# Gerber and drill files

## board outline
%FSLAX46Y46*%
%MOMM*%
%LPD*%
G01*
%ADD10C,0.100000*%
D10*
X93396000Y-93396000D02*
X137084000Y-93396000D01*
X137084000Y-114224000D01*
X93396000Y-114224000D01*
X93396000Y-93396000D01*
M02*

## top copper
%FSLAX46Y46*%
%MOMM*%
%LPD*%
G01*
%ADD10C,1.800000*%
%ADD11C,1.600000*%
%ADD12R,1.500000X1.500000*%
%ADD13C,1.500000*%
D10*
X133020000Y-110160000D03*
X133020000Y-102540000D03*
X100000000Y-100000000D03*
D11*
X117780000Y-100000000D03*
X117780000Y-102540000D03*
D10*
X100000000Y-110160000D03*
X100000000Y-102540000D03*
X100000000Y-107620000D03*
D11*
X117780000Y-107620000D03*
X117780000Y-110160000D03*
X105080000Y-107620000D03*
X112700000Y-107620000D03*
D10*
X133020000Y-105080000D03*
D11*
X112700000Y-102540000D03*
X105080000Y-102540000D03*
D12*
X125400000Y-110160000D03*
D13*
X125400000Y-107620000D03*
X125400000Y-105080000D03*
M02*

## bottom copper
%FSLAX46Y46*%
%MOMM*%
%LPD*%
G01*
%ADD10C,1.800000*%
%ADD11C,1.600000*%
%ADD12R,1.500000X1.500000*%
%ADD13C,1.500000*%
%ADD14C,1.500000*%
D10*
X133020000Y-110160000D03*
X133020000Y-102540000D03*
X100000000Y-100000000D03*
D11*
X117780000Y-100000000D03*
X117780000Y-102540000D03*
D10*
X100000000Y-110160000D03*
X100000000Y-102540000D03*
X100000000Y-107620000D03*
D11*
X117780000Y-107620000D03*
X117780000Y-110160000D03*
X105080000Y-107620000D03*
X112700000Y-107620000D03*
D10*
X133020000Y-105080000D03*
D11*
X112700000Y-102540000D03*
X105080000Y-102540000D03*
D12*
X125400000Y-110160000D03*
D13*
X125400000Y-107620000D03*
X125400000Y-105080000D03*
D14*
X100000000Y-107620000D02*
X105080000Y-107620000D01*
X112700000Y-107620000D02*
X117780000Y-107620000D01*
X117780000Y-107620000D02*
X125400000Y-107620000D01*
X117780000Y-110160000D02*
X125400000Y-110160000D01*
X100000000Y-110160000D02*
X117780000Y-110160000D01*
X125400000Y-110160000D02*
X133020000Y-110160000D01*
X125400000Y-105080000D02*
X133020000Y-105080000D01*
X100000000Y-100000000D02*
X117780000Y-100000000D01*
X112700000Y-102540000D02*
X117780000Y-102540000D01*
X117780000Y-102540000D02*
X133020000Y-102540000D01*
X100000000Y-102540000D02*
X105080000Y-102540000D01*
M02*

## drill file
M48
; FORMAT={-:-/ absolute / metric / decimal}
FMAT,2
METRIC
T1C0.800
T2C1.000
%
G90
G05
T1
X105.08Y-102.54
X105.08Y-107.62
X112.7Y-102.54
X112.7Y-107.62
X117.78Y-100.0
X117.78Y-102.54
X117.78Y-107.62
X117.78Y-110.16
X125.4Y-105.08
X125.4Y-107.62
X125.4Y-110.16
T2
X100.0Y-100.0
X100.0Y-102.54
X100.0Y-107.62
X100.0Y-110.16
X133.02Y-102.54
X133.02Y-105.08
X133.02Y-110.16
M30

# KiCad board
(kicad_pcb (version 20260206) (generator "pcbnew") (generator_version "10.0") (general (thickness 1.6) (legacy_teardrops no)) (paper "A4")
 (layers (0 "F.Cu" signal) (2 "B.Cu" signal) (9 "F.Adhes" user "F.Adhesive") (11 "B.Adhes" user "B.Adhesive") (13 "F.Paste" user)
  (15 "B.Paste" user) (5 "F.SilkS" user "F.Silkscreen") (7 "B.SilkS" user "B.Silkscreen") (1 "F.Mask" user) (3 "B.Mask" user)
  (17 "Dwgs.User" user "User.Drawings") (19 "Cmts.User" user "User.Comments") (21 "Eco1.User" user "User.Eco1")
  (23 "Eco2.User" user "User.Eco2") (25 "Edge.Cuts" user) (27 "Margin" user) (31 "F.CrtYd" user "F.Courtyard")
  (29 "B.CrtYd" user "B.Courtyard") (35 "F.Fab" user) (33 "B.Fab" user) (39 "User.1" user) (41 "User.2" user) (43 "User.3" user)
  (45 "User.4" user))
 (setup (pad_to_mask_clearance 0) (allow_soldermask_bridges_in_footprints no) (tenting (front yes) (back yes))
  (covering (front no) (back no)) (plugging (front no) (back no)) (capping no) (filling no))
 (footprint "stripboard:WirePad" (layer "F.Cu") (at 133.02 110.16)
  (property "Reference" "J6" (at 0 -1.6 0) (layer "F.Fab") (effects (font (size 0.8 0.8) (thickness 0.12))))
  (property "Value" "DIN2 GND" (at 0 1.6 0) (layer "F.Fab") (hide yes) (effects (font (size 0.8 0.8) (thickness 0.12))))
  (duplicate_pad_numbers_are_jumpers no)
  (pad "1" thru_hole circle (at 0 0) (size 1.8 1.8) (drill 1) (layers "*.Cu" "*.Mask") (remove_unused_layers no) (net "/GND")))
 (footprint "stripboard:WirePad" (layer "F.Cu") (at 133.02 102.54)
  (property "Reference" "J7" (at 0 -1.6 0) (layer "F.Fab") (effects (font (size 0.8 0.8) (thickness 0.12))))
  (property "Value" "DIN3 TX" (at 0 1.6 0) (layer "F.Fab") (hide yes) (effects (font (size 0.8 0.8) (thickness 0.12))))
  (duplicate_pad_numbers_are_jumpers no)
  (pad "1" thru_hole circle (at 0 0) (size 1.8 1.8) (drill 1) (layers "*.Cu" "*.Mask") (remove_unused_layers no) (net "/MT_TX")))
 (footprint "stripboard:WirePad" (layer "F.Cu") (at 100 100)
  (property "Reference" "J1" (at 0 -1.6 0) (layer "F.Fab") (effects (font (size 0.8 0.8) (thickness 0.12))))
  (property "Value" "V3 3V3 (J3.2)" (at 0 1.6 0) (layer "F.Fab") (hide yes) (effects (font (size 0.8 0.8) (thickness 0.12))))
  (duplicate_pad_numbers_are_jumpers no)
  (pad "1" thru_hole circle (at 0 0) (size 1.8 1.8) (drill 1) (layers "*.Cu" "*.Mask") (remove_unused_layers no) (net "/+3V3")))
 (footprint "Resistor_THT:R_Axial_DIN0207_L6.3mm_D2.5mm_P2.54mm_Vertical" (layer "F.Cu") (at 117.78 100 -90)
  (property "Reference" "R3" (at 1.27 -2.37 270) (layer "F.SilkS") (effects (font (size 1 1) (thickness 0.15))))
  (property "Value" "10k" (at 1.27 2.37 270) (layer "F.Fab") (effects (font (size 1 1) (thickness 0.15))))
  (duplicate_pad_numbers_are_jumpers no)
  (pad "1" thru_hole circle (at 0 0 270) (size 1.6 1.6) (drill 0.8) (layers "*.Cu" "*.Mask") (remove_unused_layers no) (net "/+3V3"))
  (pad "2" thru_hole circle (at 2.54 0 270) (size 1.6 1.6) (drill 0.8) (layers "*.Cu" "*.Mask") (remove_unused_layers no) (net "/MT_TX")))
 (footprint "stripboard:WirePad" (layer "F.Cu") (at 100 110.16)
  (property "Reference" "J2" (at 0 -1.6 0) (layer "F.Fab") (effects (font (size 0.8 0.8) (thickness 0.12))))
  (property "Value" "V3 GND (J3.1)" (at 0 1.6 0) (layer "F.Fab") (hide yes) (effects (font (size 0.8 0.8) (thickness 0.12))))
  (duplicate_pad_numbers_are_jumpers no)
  (pad "1" thru_hole circle (at 0 0) (size 1.8 1.8) (drill 1) (layers "*.Cu" "*.Mask") (remove_unused_layers no) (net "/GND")))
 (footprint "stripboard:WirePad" (layer "F.Cu") (at 100 102.54)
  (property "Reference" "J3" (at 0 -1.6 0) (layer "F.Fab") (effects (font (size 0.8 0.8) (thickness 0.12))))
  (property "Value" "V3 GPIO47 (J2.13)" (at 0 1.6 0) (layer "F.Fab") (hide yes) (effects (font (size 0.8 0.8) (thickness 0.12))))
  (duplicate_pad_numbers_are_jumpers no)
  (pad "1" thru_hole circle (at 0 0) (size 1.8 1.8) (drill 1) (layers "*.Cu" "*.Mask") (remove_unused_layers no) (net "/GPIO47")))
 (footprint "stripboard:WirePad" (layer "F.Cu") (at 100 107.62)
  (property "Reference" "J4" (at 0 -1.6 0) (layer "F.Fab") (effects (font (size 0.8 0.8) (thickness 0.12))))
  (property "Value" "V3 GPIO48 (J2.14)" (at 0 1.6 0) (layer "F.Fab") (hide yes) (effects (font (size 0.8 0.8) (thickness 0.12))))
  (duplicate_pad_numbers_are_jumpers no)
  (pad "1" thru_hole circle (at 0 0) (size 1.8 1.8) (drill 1) (layers "*.Cu" "*.Mask") (remove_unused_layers no) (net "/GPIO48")))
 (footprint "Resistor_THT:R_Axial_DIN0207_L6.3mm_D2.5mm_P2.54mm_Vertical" (layer "F.Cu") (at 117.78 107.62 -90)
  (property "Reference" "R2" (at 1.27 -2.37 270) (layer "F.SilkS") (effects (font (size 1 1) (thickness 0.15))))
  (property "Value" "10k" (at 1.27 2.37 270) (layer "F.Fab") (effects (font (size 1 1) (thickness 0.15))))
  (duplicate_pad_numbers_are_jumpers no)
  (pad "1" thru_hole circle (at 0 0 270) (size 1.6 1.6) (drill 0.8) (layers "*.Cu" "*.Mask") (remove_unused_layers no) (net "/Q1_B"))
  (pad "2" thru_hole circle (at 2.54 0 270) (size 1.6 1.6) (drill 0.8) (layers "*.Cu" "*.Mask") (remove_unused_layers no) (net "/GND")))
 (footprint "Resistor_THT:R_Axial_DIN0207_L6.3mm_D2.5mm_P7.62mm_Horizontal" (layer "F.Cu") (at 105.08 107.62)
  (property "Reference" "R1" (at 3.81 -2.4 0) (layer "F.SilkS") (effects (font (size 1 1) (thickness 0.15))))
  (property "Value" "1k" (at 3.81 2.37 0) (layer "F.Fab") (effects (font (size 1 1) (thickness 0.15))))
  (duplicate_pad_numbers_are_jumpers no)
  (pad "1" thru_hole circle (at 0 0) (size 1.6 1.6) (drill 0.8) (layers "*.Cu" "*.Mask") (remove_unused_layers no) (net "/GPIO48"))
  (pad "2" thru_hole circle (at 7.62 0) (size 1.6 1.6) (drill 0.8) (layers "*.Cu" "*.Mask") (remove_unused_layers no) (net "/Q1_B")))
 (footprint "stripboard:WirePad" (layer "F.Cu") (at 133.02 105.08)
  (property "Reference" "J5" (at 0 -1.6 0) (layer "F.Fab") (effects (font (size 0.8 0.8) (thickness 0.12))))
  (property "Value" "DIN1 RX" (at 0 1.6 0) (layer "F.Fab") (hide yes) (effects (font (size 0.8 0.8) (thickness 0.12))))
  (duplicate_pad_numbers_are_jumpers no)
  (pad "1" thru_hole circle (at 0 0) (size 1.8 1.8) (drill 1) (layers "*.Cu" "*.Mask") (remove_unused_layers no) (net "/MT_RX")))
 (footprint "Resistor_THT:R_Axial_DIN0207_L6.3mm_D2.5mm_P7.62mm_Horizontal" (layer "F.Cu") (at 112.7 102.54 180)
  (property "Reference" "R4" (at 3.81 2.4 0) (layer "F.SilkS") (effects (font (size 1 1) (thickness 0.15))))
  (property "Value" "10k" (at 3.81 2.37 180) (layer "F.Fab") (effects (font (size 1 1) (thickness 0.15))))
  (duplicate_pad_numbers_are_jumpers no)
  (pad "1" thru_hole circle (at 0 0 180) (size 1.6 1.6) (drill 0.8) (layers "*.Cu" "*.Mask") (remove_unused_layers no) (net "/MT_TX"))
  (pad "2" thru_hole circle (at 7.62 0 180) (size 1.6 1.6) (drill 0.8) (layers "*.Cu" "*.Mask") (remove_unused_layers no) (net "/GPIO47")))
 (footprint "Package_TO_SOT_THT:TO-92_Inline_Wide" (layer "F.Cu") (at 125.4 110.16 90)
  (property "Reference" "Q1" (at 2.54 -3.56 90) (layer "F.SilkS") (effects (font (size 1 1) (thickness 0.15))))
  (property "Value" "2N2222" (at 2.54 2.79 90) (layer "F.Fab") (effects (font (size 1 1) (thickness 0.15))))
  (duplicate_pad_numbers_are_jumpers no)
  (pad "1" thru_hole rect (at 0 0 90) (size 1.5 1.5) (drill 0.8) (layers "*.Cu" "*.Mask") (remove_unused_layers no) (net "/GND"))
  (pad "2" thru_hole circle (at 2.54 0 90) (size 1.5 1.5) (drill 0.8) (layers "*.Cu" "*.Mask") (remove_unused_layers no) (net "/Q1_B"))
  (pad "3" thru_hole circle (at 5.08 0 90) (size 1.5 1.5) (drill 0.8) (layers "*.Cu" "*.Mask") (remove_unused_layers no) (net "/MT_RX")))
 (gr_rect (start 93.396 93.396) (end 137.084 114.224) (stroke (width 0.1) (type default)) (fill no) (layer "Edge.Cuts"))
 (segment (start 100 107.62) (end 105.08 107.62) (width 1.5) (layer "B.Cu") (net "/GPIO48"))
 (segment (start 112.7 107.62) (end 117.78 107.62) (width 1.5) (layer "B.Cu") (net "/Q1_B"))
 (segment (start 117.78 107.62) (end 125.4 107.62) (width 1.5) (layer "B.Cu") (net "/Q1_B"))
 (segment (start 117.78 110.16) (end 125.4 110.16) (width 1.5) (layer "B.Cu") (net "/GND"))
 (segment (start 100 110.16) (end 117.78 110.16) (width 1.5) (layer "B.Cu") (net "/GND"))
 (segment (start 125.4 110.16) (end 133.02 110.16) (width 1.5) (layer "B.Cu") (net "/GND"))
 (segment (start 125.4 105.08) (end 133.02 105.08) (width 1.5) (layer "B.Cu") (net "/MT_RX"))
 (segment (start 100 100) (end 117.78 100) (width 1.5) (layer "B.Cu") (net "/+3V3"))
 (segment (start 112.7 102.54) (end 117.78 102.54) (width 1.5) (layer "B.Cu") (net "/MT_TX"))
 (segment (start 117.78 102.54) (end 133.02 102.54) (width 1.5) (layer "B.Cu") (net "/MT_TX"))
 (segment (start 100 102.54) (end 105.08 102.54) (width 1.5) (layer "B.Cu") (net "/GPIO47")))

